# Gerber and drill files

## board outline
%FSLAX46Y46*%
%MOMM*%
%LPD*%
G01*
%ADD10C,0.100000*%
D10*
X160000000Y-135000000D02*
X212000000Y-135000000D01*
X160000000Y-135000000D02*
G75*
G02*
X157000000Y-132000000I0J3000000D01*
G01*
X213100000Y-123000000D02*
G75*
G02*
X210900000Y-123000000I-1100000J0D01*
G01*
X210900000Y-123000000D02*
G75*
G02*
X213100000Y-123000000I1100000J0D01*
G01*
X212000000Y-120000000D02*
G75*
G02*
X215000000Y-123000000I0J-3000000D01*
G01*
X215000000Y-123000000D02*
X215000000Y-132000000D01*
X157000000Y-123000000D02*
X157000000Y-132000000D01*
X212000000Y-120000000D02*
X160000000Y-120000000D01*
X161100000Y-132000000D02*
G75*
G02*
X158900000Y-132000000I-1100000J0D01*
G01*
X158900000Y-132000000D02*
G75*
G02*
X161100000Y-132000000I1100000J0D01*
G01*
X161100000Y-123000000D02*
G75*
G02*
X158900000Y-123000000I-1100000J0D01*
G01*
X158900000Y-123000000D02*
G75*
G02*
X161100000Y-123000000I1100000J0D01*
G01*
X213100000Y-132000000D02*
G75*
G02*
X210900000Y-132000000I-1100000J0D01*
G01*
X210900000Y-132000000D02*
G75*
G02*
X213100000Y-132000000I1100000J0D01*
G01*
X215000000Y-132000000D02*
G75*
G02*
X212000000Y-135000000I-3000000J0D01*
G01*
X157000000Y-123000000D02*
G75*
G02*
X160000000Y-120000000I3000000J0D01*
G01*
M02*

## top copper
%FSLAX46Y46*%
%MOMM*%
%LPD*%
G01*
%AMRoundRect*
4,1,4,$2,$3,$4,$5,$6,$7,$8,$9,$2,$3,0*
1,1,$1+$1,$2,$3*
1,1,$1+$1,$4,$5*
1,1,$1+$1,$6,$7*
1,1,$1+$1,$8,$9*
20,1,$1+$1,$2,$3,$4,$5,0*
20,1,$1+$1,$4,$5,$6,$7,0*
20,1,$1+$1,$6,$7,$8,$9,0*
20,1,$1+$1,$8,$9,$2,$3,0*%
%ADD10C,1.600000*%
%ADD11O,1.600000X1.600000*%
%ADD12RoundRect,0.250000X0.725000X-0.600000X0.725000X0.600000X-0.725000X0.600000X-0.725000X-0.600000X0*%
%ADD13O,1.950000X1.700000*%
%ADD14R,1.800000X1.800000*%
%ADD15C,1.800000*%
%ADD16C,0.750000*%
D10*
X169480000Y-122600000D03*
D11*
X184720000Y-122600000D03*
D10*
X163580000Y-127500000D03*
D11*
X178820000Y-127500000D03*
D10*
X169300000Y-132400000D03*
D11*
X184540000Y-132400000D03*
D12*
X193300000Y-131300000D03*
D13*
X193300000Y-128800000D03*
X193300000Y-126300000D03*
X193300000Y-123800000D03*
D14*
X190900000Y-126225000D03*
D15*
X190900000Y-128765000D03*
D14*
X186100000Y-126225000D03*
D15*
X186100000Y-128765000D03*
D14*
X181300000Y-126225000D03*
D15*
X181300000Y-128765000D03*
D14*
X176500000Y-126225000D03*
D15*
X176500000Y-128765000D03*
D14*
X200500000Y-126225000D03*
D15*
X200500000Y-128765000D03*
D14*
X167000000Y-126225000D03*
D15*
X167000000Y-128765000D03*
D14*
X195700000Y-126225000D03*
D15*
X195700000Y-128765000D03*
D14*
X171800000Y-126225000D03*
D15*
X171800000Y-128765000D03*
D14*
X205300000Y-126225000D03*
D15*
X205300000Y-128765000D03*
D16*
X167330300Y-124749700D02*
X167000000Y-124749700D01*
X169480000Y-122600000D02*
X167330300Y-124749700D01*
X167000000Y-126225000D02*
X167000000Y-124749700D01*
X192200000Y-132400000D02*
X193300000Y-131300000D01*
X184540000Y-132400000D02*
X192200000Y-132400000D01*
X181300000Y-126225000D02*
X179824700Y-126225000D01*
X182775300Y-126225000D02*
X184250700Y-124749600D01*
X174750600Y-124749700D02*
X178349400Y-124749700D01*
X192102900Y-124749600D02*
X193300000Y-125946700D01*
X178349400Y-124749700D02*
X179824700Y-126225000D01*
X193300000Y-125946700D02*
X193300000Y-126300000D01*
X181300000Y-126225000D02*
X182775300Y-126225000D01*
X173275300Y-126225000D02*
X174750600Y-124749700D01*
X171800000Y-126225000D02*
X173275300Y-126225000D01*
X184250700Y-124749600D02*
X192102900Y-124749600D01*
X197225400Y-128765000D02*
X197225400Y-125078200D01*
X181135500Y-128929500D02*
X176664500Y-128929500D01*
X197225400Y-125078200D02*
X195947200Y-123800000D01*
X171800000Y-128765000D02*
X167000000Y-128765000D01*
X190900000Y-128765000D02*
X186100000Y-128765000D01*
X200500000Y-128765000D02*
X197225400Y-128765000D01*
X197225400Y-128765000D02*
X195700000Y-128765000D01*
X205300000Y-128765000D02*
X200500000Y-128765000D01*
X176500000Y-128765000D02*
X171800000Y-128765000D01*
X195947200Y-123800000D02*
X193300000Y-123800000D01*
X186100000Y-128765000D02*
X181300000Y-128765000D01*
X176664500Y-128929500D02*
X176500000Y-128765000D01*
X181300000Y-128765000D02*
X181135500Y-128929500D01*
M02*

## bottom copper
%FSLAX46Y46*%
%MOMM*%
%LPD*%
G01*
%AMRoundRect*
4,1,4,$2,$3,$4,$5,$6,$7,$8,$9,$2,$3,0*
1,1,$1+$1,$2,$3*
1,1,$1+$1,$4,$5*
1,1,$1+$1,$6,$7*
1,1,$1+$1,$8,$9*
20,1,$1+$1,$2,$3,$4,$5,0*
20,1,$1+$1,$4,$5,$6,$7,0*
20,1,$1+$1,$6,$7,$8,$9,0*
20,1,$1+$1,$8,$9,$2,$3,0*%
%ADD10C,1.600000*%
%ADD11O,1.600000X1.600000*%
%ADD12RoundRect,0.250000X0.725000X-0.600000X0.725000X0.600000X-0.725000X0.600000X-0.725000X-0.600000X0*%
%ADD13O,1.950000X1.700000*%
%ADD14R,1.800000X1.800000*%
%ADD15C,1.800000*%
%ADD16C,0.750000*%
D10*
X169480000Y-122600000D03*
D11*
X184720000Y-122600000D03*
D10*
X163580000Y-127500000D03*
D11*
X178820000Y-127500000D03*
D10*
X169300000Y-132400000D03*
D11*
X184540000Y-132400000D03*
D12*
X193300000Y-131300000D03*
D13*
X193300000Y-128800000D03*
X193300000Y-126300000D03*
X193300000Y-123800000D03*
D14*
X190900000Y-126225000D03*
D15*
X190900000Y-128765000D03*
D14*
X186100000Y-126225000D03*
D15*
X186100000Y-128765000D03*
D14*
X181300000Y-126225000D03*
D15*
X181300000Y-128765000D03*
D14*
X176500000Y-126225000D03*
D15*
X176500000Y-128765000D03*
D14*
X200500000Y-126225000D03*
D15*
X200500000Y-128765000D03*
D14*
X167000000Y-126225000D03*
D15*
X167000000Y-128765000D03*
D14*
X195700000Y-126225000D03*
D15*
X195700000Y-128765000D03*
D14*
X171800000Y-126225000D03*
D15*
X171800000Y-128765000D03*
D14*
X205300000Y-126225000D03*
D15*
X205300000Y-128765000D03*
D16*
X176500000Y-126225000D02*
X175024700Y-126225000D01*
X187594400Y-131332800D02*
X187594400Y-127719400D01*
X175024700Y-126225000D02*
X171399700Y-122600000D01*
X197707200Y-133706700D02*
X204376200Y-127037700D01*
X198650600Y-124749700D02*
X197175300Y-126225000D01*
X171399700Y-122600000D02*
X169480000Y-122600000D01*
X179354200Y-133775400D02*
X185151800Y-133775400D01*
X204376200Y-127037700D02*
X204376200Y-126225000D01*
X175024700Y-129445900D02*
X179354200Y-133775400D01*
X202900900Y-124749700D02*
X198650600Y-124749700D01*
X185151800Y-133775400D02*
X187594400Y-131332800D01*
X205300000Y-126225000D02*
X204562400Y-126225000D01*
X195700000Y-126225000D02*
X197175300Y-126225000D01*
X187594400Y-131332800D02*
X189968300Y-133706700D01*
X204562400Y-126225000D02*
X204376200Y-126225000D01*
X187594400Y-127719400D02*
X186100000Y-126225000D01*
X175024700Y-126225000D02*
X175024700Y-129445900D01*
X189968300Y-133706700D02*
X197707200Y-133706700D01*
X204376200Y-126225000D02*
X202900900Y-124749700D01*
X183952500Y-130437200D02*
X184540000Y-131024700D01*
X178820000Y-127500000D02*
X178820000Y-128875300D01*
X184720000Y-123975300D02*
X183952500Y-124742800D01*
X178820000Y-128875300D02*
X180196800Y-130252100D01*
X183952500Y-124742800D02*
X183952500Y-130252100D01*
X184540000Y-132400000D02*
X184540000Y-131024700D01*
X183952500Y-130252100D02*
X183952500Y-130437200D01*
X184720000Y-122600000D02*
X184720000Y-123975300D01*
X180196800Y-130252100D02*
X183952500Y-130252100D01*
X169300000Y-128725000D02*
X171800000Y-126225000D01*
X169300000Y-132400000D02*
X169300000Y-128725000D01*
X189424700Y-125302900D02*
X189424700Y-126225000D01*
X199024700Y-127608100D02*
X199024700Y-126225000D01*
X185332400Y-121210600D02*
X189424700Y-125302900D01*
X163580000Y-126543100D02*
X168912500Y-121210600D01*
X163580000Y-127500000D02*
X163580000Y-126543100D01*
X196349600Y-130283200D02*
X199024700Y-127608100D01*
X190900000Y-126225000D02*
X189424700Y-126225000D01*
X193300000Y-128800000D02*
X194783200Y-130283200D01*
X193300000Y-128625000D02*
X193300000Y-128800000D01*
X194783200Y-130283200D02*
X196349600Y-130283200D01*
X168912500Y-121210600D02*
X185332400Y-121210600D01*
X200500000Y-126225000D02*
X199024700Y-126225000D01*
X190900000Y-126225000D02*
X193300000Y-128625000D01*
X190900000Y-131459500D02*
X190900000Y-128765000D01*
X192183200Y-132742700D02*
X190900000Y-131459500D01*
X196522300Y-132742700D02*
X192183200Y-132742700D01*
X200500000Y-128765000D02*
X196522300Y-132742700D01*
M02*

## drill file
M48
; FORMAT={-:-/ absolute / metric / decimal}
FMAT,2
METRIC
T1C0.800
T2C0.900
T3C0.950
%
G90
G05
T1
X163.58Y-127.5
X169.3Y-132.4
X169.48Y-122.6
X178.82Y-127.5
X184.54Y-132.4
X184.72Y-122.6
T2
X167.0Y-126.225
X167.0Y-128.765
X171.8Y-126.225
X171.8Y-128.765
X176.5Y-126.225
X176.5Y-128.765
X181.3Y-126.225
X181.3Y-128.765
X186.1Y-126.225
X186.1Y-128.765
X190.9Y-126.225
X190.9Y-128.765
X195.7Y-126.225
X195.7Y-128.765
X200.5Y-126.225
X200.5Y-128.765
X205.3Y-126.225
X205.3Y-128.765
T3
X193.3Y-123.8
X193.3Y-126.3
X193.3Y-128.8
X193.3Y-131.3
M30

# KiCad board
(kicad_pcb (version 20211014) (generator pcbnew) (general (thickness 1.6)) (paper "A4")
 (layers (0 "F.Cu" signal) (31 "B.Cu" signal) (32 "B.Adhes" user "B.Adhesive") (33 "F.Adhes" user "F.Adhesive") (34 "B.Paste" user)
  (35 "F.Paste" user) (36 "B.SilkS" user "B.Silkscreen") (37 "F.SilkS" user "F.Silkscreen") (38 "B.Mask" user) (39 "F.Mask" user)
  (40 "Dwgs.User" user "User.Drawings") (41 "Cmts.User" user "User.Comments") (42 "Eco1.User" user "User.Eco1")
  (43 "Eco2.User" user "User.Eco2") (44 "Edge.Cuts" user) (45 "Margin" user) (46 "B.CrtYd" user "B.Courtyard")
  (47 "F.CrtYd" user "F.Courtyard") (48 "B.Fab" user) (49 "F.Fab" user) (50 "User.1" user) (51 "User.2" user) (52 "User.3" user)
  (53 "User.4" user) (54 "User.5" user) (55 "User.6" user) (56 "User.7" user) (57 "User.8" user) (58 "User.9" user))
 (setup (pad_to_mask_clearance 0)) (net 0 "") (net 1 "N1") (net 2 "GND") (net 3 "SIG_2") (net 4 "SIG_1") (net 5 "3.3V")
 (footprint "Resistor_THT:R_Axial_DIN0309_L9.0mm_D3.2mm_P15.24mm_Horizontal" (layer "F.Cu") (at 169.48 122.6)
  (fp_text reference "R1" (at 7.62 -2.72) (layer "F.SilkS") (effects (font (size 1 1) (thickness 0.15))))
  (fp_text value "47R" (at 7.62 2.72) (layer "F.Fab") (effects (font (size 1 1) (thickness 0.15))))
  (pad "1" thru_hole circle (at 0 0) (size 1.6 1.6) (drill 0.8) (layers *.Cu *.Mask) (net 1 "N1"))
  (pad "2" thru_hole oval (at 15.24 0) (size 1.6 1.6) (drill 0.8) (layers *.Cu *.Mask) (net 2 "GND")))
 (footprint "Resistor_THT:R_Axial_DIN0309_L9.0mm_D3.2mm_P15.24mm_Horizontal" (layer "F.Cu") (at 163.58 127.5)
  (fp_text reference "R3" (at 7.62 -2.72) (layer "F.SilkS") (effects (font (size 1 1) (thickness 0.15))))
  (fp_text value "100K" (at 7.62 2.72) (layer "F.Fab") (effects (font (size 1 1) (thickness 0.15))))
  (pad "1" thru_hole circle (at 0 0) (size 1.6 1.6) (drill 0.8) (layers *.Cu *.Mask) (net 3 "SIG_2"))
  (pad "2" thru_hole oval (at 15.24 0) (size 1.6 1.6) (drill 0.8) (layers *.Cu *.Mask) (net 2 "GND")))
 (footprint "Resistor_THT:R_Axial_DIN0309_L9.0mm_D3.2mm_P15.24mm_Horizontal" (layer "F.Cu") (at 169.3 132.4)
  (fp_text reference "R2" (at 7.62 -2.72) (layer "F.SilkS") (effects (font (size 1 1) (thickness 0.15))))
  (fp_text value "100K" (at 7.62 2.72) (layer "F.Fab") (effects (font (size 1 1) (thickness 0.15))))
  (pad "1" thru_hole circle (at 0 0) (size 1.6 1.6) (drill 0.8) (layers *.Cu *.Mask) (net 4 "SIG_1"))
  (pad "2" thru_hole oval (at 15.24 0) (size 1.6 1.6) (drill 0.8) (layers *.Cu *.Mask) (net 2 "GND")))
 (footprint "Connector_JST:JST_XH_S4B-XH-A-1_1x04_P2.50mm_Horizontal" (layer "F.Cu") (at 193.3 131.3 90)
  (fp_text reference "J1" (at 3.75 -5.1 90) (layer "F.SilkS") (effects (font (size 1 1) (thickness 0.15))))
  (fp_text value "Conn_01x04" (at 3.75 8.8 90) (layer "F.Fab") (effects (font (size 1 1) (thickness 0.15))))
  (pad "1" thru_hole roundrect (at 0 0 90) (size 1.7 1.95) (drill 0.95) (layers *.Cu *.Mask) (roundrect_rratio 0.1470588235) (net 2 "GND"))
  (pad "2" thru_hole oval (at 2.5 0 90) (size 1.7 1.95) (drill 0.95) (layers *.Cu *.Mask) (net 3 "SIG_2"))
  (pad "3" thru_hole oval (at 5 0 90) (size 1.7 1.95) (drill 0.95) (layers *.Cu *.Mask) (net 4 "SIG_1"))
  (pad "4" thru_hole oval (at 7.5 0 90) (size 1.7 1.95) (drill 0.95) (layers *.Cu *.Mask) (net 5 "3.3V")))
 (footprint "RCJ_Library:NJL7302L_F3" (layer "B.Cu") (at 190.9 126.225 -90)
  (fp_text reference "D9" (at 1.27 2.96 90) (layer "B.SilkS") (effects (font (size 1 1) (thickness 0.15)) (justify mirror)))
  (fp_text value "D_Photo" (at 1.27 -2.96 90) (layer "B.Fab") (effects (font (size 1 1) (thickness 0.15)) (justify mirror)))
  (pad "1" thru_hole rect (at 0 0 270) (size 1.8 1.8) (drill 0.9) (layers *.Cu *.Mask) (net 3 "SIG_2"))
  (pad "2" thru_hole circle (at 2.54 0 270) (size 1.8 1.8) (drill 0.9) (layers *.Cu *.Mask) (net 5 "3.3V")))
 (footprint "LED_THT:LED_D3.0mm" (layer "B.Cu") (at 186.1 126.225 -90)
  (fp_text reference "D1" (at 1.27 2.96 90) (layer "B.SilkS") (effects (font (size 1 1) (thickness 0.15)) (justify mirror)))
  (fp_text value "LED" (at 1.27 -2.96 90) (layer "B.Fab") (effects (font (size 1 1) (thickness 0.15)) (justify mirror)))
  (pad "1" thru_hole rect (at 0 0 270) (size 1.8 1.8) (drill 0.9) (layers *.Cu *.Mask) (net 1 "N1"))
  (pad "2" thru_hole circle (at 2.54 0 270) (size 1.8 1.8) (drill 0.9) (layers *.Cu *.Mask) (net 5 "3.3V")))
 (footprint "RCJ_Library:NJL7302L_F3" (layer "B.Cu") (at 181.3 126.225 -90)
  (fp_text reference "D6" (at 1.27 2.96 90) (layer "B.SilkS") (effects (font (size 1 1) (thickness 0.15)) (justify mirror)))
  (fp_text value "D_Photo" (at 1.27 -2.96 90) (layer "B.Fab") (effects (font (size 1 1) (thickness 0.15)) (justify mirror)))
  (pad "1" thru_hole rect (at 0 0 270) (size 1.8 1.8) (drill 0.9) (layers *.Cu *.Mask) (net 4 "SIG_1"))
  (pad "2" thru_hole circle (at 2.54 0 270) (size 1.8 1.8) (drill 0.9) (layers *.Cu *.Mask) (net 5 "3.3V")))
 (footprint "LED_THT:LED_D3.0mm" (layer "B.Cu") (at 176.5 126.225 -90)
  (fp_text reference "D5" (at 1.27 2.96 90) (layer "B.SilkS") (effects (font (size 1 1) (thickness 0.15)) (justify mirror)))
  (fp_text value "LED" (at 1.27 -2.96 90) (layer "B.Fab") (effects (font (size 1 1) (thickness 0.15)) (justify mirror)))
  (pad "1" thru_hole rect (at 0 0 270) (size 1.8 1.8) (drill 0.9) (layers *.Cu *.Mask) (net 1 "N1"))
  (pad "2" thru_hole circle (at 2.54 0 270) (size 1.8 1.8) (drill 0.9) (layers *.Cu *.Mask) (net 5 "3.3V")))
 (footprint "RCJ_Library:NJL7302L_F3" (layer "B.Cu") (at 200.5 126.225 -90)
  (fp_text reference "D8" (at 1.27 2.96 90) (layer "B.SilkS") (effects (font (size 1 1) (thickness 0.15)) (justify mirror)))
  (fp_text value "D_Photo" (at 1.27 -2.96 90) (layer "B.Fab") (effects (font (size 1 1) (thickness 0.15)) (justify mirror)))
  (pad "1" thru_hole rect (at 0 0 270) (size 1.8 1.8) (drill 0.9) (layers *.Cu *.Mask) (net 3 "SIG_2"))
  (pad "2" thru_hole circle (at 2.54 0 270) (size 1.8 1.8) (drill 0.9) (layers *.Cu *.Mask) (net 5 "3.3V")))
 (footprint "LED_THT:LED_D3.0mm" (layer "B.Cu") (at 167 126.225 -90)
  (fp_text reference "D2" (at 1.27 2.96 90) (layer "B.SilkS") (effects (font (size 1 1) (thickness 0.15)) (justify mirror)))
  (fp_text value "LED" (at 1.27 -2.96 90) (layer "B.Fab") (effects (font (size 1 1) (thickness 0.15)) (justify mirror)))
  (pad "1" thru_hole rect (at 0 0 270) (size 1.8 1.8) (drill 0.9) (layers *.Cu *.Mask) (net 1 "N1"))
  (pad "2" thru_hole circle (at 2.54 0 270) (size 1.8 1.8) (drill 0.9) (layers *.Cu *.Mask) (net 5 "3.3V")))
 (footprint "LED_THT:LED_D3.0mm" (layer "B.Cu") (at 195.7 126.225 -90)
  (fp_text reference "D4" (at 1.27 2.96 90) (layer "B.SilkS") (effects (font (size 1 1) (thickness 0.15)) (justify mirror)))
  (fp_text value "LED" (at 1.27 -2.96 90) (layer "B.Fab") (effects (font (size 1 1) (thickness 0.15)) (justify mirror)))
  (pad "1" thru_hole rect (at 0 0 270) (size 1.8 1.8) (drill 0.9) (layers *.Cu *.Mask) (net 1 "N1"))
  (pad "2" thru_hole circle (at 2.54 0 270) (size 1.8 1.8) (drill 0.9) (layers *.Cu *.Mask) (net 5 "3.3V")))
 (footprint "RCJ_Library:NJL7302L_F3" (layer "B.Cu") (at 171.8 126.225 -90)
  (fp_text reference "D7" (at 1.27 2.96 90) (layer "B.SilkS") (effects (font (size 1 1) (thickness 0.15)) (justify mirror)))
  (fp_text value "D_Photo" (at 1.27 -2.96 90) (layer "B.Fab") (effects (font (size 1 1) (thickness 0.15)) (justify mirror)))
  (pad "1" thru_hole rect (at 0 0 270) (size 1.8 1.8) (drill 0.9) (layers *.Cu *.Mask) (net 4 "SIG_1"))
  (pad "2" thru_hole circle (at 2.54 0 270) (size 1.8 1.8) (drill 0.9) (layers *.Cu *.Mask) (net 5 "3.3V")))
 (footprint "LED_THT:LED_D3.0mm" (layer "B.Cu") (at 205.3 126.225 -90)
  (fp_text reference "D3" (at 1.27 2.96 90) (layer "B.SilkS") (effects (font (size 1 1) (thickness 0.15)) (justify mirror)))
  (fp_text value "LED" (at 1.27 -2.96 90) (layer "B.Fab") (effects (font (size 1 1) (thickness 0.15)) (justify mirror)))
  (pad "1" thru_hole rect (at 0 0 270) (size 1.8 1.8) (drill 0.9) (layers *.Cu *.Mask) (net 1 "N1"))
  (pad "2" thru_hole circle (at 2.54 0 270) (size 1.8 1.8) (drill 0.9) (layers *.Cu *.Mask) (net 5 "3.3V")))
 (gr_line (start 160 135) (end 212 135) (layer "Edge.Cuts") (width 0.1))
 (gr_arc (start 160 135) (mid 157.87868 134.12132) (end 157 132) (layer "Edge.Cuts") (width 0.1))
 (gr_circle (center 212 123) (end 213.1 123) (layer "Edge.Cuts") (width 0.1) (fill none))
 (gr_arc (start 212 120) (mid 214.12132 120.87868) (end 215 123) (layer "Edge.Cuts") (width 0.1))
 (gr_line (start 215 123) (end 215 132) (layer "Edge.Cuts") (width 0.1))
 (gr_line (start 157 123) (end 157 132) (layer "Edge.Cuts") (width 0.1))
 (gr_line (start 212 120) (end 160 120) (layer "Edge.Cuts") (width 0.1))
 (gr_circle (center 160 132) (end 161.1 132) (layer "Edge.Cuts") (width 0.1) (fill none))
 (gr_circle (center 160 123) (end 161.1 123) (layer "Edge.Cuts") (width 0.1) (fill none))
 (gr_circle (center 212 132) (end 213.1 132) (layer "Edge.Cuts") (width 0.1) (fill none))
 (gr_arc (start 215 132) (mid 214.12132 134.12132) (end 212 135) (layer "Edge.Cuts") (width 0.1))
 (gr_arc (start 157 123) (mid 157.87868 120.87868) (end 160 120) (layer "Edge.Cuts") (width 0.1))
 (segment (start 167.3303 124.7497) (end 167 124.7497) (width 0.75) (layer "F.Cu") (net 1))
 (segment (start 169.48 122.6) (end 167.3303 124.7497) (width 0.75) (layer "F.Cu") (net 1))
 (segment (start 167 126.225) (end 167 124.7497) (width 0.75) (layer "F.Cu") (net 1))
 (segment (start 176.5 126.225) (end 175.0247 126.225) (width 0.75) (layer "B.Cu") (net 1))
 (segment (start 187.5944 131.3328) (end 187.5944 127.7194) (width 0.75) (layer "B.Cu") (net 1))
 (segment (start 175.0247 126.225) (end 171.3997 122.6) (width 0.75) (layer "B.Cu") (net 1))
 (segment (start 197.7072 133.7067) (end 204.3762 127.0377) (width 0.75) (layer "B.Cu") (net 1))
 (segment (start 198.6506 124.7497) (end 197.1753 126.225) (width 0.75) (layer "B.Cu") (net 1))
 (segment (start 171.3997 122.6) (end 169.48 122.6) (width 0.75) (layer "B.Cu") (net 1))
 (segment (start 179.3542 133.7754) (end 185.1518 133.7754) (width 0.75) (layer "B.Cu") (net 1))
 (segment (start 204.3762 127.0377) (end 204.3762 126.225) (width 0.75) (layer "B.Cu") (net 1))
 (segment (start 175.0247 129.4459) (end 179.3542 133.7754) (width 0.75) (layer "B.Cu") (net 1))
 (segment (start 202.9009 124.7497) (end 198.6506 124.7497) (width 0.75) (layer "B.Cu") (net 1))
 (segment (start 185.1518 133.7754) (end 187.5944 131.3328) (width 0.75) (layer "B.Cu") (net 1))
 (segment (start 205.3 126.225) (end 204.5624 126.225) (width 0.75) (layer "B.Cu") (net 1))
 (segment (start 195.7 126.225) (end 197.1753 126.225) (width 0.75) (layer "B.Cu") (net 1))
 (segment (start 187.5944 131.3328) (end 189.9683 133.7067) (width 0.75) (layer "B.Cu") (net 1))
 (segment (start 204.5624 126.225) (end 204.3762 126.225) (width 0.75) (layer "B.Cu") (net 1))
 (segment (start 187.5944 127.7194) (end 186.1 126.225) (width 0.75) (layer "B.Cu") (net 1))
 (segment (start 175.0247 126.225) (end 175.0247 129.4459) (width 0.75) (layer "B.Cu") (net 1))
 (segment (start 189.9683 133.7067) (end 197.7072 133.7067) (width 0.75) (layer "B.Cu") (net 1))
 (segment (start 204.3762 126.225) (end 202.9009 124.7497) (width 0.75) (layer "B.Cu") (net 1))
 (segment (start 192.2 132.4) (end 193.3 131.3) (width 0.75) (layer "F.Cu") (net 2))
 (segment (start 184.54 132.4) (end 192.2 132.4) (width 0.75) (layer "F.Cu") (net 2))
 (segment (start 183.9525 130.4372) (end 184.54 131.0247) (width 0.75) (layer "B.Cu") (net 2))
 (segment (start 178.82 127.5) (end 178.82 128.8753) (width 0.75) (layer "B.Cu") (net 2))
 (segment (start 184.72 123.9753) (end 183.9525 124.7428) (width 0.75) (layer "B.Cu") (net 2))
 (segment (start 178.82 128.8753) (end 180.1968 130.2521) (width 0.75) (layer "B.Cu") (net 2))
 (segment (start 183.9525 124.7428) (end 183.9525 130.2521) (width 0.75) (layer "B.Cu") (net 2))
 (segment (start 184.54 132.4) (end 184.54 131.0247) (width 0.75) (layer "B.Cu") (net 2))
 (segment (start 183.9525 130.2521) (end 183.9525 130.4372) (width 0.75) (layer "B.Cu") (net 2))
 (segment (start 184.72 122.6) (end 184.72 123.9753) (width 0.75) (layer "B.Cu") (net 2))
 (segment (start 180.1968 130.2521) (end 183.9525 130.2521) (width 0.75) (layer "B.Cu") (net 2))
 (segment (start 181.3 126.225) (end 179.8247 126.225) (width 0.75) (layer "F.Cu") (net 4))
 (segment (start 182.7753 126.225) (end 184.2507 124.7496) (width 0.75) (layer "F.Cu") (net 4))
 (segment (start 174.7506 124.7497) (end 178.3494 124.7497) (width 0.75) (layer "F.Cu") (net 4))
 (segment (start 192.1029 124.7496) (end 193.3 125.9467) (width 0.75) (layer "F.Cu") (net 4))
 (segment (start 178.3494 124.7497) (end 179.8247 126.225) (width 0.75) (layer "F.Cu") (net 4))
 (segment (start 193.3 125.9467) (end 193.3 126.3) (width 0.75) (layer "F.Cu") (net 4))
 (segment (start 181.3 126.225) (end 182.7753 126.225) (width 0.75) (layer "F.Cu") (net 4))
 (segment (start 173.2753 126.225) (end 174.7506 124.7497) (width 0.75) (layer "F.Cu") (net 4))
 (segment (start 171.8 126.225) (end 173.2753 126.225) (width 0.75) (layer "F.Cu") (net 4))
 (segment (start 184.2507 124.7496) (end 192.1029 124.7496) (width 0.75) (layer "F.Cu") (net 4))
 (segment (start 169.3 128.725) (end 171.8 126.225) (width 0.75) (layer "B.Cu") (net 4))
 (segment (start 169.3 132.4) (end 169.3 128.725) (width 0.75) (layer "B.Cu") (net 4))
 (segment (start 189.4247 125.3029) (end 189.4247 126.225) (width 0.75) (layer "B.Cu") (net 3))
 (segment (start 199.0247 127.6081) (end 199.0247 126.225) (width 0.75) (layer "B.Cu") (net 3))
 (segment (start 185.3324 121.2106) (end 189.4247 125.3029) (width 0.75) (layer "B.Cu") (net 3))
 (segment (start 163.58 126.5431) (end 168.9125 121.2106) (width 0.75) (layer "B.Cu") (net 3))
 (segment (start 163.58 127.5) (end 163.58 126.5431) (width 0.75) (layer "B.Cu") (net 3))
 (segment (start 196.3496 130.2832) (end 199.0247 127.6081) (width 0.75) (layer "B.Cu") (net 3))
 (segment (start 190.9 126.225) (end 189.4247 126.225) (width 0.75) (layer "B.Cu") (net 3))
 (segment (start 193.3 128.8) (end 194.7832 130.2832) (width 0.75) (layer "B.Cu") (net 3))
 (segment (start 193.3 128.625) (end 193.3 128.8) (width 0.75) (layer "B.Cu") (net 3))
 (segment (start 194.7832 130.2832) (end 196.3496 130.2832) (width 0.75) (layer "B.Cu") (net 3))
 (segment (start 168.9125 121.2106) (end 185.3324 121.2106) (width 0.75) (layer "B.Cu") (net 3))
 (segment (start 200.5 126.225) (end 199.0247 126.225) (width 0.75) (layer "B.Cu") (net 3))
 (segment (start 190.9 126.225) (end 193.3 128.625) (width 0.75) (layer "B.Cu") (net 3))
 (segment (start 197.2254 128.765) (end 197.2254 125.0782) (width 0.75) (layer "F.Cu") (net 5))
 (segment (start 181.1355 128.9295) (end 176.6645 128.9295) (width 0.75) (layer "F.Cu") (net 5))
 (segment (start 197.2254 125.0782) (end 195.9472 123.8) (width 0.75) (layer "F.Cu") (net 5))
 (segment (start 171.8 128.765) (end 167 128.765) (width 0.75) (layer "F.Cu") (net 5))
 (segment (start 190.9 128.765) (end 186.1 128.765) (width 0.75) (layer "F.Cu") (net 5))
 (segment (start 200.5 128.765) (end 197.2254 128.765) (width 0.75) (layer "F.Cu") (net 5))
 (segment (start 197.2254 128.765) (end 195.7 128.765) (width 0.75) (layer "F.Cu") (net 5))
 (segment (start 205.3 128.765) (end 200.5 128.765) (width 0.75) (layer "F.Cu") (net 5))
 (segment (start 176.5 128.765) (end 171.8 128.765) (width 0.75) (layer "F.Cu") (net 5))
 (segment (start 195.9472 123.8) (end 193.3 123.8) (width 0.75) (layer "F.Cu") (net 5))
 (segment (start 186.1 128.765) (end 181.3 128.765) (width 0.75) (layer "F.Cu") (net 5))
 (segment (start 176.6645 128.9295) (end 176.5 128.765) (width 0.75) (layer "F.Cu") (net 5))
 (segment (start 181.3 128.765) (end 181.1355 128.9295) (width 0.75) (layer "F.Cu") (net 5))
 (segment (start 190.9 131.4595) (end 190.9 128.765) (width 0.75) (layer "B.Cu") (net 5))
 (segment (start 192.1832 132.7427) (end 190.9 131.4595) (width 0.75) (layer "B.Cu") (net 5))
 (segment (start 196.5223 132.7427) (end 192.1832 132.7427) (width 0.75) (layer "B.Cu") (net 5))
 (segment (start 200.5 128.765) (end 196.5223 132.7427) (width 0.75) (layer "B.Cu") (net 5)))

